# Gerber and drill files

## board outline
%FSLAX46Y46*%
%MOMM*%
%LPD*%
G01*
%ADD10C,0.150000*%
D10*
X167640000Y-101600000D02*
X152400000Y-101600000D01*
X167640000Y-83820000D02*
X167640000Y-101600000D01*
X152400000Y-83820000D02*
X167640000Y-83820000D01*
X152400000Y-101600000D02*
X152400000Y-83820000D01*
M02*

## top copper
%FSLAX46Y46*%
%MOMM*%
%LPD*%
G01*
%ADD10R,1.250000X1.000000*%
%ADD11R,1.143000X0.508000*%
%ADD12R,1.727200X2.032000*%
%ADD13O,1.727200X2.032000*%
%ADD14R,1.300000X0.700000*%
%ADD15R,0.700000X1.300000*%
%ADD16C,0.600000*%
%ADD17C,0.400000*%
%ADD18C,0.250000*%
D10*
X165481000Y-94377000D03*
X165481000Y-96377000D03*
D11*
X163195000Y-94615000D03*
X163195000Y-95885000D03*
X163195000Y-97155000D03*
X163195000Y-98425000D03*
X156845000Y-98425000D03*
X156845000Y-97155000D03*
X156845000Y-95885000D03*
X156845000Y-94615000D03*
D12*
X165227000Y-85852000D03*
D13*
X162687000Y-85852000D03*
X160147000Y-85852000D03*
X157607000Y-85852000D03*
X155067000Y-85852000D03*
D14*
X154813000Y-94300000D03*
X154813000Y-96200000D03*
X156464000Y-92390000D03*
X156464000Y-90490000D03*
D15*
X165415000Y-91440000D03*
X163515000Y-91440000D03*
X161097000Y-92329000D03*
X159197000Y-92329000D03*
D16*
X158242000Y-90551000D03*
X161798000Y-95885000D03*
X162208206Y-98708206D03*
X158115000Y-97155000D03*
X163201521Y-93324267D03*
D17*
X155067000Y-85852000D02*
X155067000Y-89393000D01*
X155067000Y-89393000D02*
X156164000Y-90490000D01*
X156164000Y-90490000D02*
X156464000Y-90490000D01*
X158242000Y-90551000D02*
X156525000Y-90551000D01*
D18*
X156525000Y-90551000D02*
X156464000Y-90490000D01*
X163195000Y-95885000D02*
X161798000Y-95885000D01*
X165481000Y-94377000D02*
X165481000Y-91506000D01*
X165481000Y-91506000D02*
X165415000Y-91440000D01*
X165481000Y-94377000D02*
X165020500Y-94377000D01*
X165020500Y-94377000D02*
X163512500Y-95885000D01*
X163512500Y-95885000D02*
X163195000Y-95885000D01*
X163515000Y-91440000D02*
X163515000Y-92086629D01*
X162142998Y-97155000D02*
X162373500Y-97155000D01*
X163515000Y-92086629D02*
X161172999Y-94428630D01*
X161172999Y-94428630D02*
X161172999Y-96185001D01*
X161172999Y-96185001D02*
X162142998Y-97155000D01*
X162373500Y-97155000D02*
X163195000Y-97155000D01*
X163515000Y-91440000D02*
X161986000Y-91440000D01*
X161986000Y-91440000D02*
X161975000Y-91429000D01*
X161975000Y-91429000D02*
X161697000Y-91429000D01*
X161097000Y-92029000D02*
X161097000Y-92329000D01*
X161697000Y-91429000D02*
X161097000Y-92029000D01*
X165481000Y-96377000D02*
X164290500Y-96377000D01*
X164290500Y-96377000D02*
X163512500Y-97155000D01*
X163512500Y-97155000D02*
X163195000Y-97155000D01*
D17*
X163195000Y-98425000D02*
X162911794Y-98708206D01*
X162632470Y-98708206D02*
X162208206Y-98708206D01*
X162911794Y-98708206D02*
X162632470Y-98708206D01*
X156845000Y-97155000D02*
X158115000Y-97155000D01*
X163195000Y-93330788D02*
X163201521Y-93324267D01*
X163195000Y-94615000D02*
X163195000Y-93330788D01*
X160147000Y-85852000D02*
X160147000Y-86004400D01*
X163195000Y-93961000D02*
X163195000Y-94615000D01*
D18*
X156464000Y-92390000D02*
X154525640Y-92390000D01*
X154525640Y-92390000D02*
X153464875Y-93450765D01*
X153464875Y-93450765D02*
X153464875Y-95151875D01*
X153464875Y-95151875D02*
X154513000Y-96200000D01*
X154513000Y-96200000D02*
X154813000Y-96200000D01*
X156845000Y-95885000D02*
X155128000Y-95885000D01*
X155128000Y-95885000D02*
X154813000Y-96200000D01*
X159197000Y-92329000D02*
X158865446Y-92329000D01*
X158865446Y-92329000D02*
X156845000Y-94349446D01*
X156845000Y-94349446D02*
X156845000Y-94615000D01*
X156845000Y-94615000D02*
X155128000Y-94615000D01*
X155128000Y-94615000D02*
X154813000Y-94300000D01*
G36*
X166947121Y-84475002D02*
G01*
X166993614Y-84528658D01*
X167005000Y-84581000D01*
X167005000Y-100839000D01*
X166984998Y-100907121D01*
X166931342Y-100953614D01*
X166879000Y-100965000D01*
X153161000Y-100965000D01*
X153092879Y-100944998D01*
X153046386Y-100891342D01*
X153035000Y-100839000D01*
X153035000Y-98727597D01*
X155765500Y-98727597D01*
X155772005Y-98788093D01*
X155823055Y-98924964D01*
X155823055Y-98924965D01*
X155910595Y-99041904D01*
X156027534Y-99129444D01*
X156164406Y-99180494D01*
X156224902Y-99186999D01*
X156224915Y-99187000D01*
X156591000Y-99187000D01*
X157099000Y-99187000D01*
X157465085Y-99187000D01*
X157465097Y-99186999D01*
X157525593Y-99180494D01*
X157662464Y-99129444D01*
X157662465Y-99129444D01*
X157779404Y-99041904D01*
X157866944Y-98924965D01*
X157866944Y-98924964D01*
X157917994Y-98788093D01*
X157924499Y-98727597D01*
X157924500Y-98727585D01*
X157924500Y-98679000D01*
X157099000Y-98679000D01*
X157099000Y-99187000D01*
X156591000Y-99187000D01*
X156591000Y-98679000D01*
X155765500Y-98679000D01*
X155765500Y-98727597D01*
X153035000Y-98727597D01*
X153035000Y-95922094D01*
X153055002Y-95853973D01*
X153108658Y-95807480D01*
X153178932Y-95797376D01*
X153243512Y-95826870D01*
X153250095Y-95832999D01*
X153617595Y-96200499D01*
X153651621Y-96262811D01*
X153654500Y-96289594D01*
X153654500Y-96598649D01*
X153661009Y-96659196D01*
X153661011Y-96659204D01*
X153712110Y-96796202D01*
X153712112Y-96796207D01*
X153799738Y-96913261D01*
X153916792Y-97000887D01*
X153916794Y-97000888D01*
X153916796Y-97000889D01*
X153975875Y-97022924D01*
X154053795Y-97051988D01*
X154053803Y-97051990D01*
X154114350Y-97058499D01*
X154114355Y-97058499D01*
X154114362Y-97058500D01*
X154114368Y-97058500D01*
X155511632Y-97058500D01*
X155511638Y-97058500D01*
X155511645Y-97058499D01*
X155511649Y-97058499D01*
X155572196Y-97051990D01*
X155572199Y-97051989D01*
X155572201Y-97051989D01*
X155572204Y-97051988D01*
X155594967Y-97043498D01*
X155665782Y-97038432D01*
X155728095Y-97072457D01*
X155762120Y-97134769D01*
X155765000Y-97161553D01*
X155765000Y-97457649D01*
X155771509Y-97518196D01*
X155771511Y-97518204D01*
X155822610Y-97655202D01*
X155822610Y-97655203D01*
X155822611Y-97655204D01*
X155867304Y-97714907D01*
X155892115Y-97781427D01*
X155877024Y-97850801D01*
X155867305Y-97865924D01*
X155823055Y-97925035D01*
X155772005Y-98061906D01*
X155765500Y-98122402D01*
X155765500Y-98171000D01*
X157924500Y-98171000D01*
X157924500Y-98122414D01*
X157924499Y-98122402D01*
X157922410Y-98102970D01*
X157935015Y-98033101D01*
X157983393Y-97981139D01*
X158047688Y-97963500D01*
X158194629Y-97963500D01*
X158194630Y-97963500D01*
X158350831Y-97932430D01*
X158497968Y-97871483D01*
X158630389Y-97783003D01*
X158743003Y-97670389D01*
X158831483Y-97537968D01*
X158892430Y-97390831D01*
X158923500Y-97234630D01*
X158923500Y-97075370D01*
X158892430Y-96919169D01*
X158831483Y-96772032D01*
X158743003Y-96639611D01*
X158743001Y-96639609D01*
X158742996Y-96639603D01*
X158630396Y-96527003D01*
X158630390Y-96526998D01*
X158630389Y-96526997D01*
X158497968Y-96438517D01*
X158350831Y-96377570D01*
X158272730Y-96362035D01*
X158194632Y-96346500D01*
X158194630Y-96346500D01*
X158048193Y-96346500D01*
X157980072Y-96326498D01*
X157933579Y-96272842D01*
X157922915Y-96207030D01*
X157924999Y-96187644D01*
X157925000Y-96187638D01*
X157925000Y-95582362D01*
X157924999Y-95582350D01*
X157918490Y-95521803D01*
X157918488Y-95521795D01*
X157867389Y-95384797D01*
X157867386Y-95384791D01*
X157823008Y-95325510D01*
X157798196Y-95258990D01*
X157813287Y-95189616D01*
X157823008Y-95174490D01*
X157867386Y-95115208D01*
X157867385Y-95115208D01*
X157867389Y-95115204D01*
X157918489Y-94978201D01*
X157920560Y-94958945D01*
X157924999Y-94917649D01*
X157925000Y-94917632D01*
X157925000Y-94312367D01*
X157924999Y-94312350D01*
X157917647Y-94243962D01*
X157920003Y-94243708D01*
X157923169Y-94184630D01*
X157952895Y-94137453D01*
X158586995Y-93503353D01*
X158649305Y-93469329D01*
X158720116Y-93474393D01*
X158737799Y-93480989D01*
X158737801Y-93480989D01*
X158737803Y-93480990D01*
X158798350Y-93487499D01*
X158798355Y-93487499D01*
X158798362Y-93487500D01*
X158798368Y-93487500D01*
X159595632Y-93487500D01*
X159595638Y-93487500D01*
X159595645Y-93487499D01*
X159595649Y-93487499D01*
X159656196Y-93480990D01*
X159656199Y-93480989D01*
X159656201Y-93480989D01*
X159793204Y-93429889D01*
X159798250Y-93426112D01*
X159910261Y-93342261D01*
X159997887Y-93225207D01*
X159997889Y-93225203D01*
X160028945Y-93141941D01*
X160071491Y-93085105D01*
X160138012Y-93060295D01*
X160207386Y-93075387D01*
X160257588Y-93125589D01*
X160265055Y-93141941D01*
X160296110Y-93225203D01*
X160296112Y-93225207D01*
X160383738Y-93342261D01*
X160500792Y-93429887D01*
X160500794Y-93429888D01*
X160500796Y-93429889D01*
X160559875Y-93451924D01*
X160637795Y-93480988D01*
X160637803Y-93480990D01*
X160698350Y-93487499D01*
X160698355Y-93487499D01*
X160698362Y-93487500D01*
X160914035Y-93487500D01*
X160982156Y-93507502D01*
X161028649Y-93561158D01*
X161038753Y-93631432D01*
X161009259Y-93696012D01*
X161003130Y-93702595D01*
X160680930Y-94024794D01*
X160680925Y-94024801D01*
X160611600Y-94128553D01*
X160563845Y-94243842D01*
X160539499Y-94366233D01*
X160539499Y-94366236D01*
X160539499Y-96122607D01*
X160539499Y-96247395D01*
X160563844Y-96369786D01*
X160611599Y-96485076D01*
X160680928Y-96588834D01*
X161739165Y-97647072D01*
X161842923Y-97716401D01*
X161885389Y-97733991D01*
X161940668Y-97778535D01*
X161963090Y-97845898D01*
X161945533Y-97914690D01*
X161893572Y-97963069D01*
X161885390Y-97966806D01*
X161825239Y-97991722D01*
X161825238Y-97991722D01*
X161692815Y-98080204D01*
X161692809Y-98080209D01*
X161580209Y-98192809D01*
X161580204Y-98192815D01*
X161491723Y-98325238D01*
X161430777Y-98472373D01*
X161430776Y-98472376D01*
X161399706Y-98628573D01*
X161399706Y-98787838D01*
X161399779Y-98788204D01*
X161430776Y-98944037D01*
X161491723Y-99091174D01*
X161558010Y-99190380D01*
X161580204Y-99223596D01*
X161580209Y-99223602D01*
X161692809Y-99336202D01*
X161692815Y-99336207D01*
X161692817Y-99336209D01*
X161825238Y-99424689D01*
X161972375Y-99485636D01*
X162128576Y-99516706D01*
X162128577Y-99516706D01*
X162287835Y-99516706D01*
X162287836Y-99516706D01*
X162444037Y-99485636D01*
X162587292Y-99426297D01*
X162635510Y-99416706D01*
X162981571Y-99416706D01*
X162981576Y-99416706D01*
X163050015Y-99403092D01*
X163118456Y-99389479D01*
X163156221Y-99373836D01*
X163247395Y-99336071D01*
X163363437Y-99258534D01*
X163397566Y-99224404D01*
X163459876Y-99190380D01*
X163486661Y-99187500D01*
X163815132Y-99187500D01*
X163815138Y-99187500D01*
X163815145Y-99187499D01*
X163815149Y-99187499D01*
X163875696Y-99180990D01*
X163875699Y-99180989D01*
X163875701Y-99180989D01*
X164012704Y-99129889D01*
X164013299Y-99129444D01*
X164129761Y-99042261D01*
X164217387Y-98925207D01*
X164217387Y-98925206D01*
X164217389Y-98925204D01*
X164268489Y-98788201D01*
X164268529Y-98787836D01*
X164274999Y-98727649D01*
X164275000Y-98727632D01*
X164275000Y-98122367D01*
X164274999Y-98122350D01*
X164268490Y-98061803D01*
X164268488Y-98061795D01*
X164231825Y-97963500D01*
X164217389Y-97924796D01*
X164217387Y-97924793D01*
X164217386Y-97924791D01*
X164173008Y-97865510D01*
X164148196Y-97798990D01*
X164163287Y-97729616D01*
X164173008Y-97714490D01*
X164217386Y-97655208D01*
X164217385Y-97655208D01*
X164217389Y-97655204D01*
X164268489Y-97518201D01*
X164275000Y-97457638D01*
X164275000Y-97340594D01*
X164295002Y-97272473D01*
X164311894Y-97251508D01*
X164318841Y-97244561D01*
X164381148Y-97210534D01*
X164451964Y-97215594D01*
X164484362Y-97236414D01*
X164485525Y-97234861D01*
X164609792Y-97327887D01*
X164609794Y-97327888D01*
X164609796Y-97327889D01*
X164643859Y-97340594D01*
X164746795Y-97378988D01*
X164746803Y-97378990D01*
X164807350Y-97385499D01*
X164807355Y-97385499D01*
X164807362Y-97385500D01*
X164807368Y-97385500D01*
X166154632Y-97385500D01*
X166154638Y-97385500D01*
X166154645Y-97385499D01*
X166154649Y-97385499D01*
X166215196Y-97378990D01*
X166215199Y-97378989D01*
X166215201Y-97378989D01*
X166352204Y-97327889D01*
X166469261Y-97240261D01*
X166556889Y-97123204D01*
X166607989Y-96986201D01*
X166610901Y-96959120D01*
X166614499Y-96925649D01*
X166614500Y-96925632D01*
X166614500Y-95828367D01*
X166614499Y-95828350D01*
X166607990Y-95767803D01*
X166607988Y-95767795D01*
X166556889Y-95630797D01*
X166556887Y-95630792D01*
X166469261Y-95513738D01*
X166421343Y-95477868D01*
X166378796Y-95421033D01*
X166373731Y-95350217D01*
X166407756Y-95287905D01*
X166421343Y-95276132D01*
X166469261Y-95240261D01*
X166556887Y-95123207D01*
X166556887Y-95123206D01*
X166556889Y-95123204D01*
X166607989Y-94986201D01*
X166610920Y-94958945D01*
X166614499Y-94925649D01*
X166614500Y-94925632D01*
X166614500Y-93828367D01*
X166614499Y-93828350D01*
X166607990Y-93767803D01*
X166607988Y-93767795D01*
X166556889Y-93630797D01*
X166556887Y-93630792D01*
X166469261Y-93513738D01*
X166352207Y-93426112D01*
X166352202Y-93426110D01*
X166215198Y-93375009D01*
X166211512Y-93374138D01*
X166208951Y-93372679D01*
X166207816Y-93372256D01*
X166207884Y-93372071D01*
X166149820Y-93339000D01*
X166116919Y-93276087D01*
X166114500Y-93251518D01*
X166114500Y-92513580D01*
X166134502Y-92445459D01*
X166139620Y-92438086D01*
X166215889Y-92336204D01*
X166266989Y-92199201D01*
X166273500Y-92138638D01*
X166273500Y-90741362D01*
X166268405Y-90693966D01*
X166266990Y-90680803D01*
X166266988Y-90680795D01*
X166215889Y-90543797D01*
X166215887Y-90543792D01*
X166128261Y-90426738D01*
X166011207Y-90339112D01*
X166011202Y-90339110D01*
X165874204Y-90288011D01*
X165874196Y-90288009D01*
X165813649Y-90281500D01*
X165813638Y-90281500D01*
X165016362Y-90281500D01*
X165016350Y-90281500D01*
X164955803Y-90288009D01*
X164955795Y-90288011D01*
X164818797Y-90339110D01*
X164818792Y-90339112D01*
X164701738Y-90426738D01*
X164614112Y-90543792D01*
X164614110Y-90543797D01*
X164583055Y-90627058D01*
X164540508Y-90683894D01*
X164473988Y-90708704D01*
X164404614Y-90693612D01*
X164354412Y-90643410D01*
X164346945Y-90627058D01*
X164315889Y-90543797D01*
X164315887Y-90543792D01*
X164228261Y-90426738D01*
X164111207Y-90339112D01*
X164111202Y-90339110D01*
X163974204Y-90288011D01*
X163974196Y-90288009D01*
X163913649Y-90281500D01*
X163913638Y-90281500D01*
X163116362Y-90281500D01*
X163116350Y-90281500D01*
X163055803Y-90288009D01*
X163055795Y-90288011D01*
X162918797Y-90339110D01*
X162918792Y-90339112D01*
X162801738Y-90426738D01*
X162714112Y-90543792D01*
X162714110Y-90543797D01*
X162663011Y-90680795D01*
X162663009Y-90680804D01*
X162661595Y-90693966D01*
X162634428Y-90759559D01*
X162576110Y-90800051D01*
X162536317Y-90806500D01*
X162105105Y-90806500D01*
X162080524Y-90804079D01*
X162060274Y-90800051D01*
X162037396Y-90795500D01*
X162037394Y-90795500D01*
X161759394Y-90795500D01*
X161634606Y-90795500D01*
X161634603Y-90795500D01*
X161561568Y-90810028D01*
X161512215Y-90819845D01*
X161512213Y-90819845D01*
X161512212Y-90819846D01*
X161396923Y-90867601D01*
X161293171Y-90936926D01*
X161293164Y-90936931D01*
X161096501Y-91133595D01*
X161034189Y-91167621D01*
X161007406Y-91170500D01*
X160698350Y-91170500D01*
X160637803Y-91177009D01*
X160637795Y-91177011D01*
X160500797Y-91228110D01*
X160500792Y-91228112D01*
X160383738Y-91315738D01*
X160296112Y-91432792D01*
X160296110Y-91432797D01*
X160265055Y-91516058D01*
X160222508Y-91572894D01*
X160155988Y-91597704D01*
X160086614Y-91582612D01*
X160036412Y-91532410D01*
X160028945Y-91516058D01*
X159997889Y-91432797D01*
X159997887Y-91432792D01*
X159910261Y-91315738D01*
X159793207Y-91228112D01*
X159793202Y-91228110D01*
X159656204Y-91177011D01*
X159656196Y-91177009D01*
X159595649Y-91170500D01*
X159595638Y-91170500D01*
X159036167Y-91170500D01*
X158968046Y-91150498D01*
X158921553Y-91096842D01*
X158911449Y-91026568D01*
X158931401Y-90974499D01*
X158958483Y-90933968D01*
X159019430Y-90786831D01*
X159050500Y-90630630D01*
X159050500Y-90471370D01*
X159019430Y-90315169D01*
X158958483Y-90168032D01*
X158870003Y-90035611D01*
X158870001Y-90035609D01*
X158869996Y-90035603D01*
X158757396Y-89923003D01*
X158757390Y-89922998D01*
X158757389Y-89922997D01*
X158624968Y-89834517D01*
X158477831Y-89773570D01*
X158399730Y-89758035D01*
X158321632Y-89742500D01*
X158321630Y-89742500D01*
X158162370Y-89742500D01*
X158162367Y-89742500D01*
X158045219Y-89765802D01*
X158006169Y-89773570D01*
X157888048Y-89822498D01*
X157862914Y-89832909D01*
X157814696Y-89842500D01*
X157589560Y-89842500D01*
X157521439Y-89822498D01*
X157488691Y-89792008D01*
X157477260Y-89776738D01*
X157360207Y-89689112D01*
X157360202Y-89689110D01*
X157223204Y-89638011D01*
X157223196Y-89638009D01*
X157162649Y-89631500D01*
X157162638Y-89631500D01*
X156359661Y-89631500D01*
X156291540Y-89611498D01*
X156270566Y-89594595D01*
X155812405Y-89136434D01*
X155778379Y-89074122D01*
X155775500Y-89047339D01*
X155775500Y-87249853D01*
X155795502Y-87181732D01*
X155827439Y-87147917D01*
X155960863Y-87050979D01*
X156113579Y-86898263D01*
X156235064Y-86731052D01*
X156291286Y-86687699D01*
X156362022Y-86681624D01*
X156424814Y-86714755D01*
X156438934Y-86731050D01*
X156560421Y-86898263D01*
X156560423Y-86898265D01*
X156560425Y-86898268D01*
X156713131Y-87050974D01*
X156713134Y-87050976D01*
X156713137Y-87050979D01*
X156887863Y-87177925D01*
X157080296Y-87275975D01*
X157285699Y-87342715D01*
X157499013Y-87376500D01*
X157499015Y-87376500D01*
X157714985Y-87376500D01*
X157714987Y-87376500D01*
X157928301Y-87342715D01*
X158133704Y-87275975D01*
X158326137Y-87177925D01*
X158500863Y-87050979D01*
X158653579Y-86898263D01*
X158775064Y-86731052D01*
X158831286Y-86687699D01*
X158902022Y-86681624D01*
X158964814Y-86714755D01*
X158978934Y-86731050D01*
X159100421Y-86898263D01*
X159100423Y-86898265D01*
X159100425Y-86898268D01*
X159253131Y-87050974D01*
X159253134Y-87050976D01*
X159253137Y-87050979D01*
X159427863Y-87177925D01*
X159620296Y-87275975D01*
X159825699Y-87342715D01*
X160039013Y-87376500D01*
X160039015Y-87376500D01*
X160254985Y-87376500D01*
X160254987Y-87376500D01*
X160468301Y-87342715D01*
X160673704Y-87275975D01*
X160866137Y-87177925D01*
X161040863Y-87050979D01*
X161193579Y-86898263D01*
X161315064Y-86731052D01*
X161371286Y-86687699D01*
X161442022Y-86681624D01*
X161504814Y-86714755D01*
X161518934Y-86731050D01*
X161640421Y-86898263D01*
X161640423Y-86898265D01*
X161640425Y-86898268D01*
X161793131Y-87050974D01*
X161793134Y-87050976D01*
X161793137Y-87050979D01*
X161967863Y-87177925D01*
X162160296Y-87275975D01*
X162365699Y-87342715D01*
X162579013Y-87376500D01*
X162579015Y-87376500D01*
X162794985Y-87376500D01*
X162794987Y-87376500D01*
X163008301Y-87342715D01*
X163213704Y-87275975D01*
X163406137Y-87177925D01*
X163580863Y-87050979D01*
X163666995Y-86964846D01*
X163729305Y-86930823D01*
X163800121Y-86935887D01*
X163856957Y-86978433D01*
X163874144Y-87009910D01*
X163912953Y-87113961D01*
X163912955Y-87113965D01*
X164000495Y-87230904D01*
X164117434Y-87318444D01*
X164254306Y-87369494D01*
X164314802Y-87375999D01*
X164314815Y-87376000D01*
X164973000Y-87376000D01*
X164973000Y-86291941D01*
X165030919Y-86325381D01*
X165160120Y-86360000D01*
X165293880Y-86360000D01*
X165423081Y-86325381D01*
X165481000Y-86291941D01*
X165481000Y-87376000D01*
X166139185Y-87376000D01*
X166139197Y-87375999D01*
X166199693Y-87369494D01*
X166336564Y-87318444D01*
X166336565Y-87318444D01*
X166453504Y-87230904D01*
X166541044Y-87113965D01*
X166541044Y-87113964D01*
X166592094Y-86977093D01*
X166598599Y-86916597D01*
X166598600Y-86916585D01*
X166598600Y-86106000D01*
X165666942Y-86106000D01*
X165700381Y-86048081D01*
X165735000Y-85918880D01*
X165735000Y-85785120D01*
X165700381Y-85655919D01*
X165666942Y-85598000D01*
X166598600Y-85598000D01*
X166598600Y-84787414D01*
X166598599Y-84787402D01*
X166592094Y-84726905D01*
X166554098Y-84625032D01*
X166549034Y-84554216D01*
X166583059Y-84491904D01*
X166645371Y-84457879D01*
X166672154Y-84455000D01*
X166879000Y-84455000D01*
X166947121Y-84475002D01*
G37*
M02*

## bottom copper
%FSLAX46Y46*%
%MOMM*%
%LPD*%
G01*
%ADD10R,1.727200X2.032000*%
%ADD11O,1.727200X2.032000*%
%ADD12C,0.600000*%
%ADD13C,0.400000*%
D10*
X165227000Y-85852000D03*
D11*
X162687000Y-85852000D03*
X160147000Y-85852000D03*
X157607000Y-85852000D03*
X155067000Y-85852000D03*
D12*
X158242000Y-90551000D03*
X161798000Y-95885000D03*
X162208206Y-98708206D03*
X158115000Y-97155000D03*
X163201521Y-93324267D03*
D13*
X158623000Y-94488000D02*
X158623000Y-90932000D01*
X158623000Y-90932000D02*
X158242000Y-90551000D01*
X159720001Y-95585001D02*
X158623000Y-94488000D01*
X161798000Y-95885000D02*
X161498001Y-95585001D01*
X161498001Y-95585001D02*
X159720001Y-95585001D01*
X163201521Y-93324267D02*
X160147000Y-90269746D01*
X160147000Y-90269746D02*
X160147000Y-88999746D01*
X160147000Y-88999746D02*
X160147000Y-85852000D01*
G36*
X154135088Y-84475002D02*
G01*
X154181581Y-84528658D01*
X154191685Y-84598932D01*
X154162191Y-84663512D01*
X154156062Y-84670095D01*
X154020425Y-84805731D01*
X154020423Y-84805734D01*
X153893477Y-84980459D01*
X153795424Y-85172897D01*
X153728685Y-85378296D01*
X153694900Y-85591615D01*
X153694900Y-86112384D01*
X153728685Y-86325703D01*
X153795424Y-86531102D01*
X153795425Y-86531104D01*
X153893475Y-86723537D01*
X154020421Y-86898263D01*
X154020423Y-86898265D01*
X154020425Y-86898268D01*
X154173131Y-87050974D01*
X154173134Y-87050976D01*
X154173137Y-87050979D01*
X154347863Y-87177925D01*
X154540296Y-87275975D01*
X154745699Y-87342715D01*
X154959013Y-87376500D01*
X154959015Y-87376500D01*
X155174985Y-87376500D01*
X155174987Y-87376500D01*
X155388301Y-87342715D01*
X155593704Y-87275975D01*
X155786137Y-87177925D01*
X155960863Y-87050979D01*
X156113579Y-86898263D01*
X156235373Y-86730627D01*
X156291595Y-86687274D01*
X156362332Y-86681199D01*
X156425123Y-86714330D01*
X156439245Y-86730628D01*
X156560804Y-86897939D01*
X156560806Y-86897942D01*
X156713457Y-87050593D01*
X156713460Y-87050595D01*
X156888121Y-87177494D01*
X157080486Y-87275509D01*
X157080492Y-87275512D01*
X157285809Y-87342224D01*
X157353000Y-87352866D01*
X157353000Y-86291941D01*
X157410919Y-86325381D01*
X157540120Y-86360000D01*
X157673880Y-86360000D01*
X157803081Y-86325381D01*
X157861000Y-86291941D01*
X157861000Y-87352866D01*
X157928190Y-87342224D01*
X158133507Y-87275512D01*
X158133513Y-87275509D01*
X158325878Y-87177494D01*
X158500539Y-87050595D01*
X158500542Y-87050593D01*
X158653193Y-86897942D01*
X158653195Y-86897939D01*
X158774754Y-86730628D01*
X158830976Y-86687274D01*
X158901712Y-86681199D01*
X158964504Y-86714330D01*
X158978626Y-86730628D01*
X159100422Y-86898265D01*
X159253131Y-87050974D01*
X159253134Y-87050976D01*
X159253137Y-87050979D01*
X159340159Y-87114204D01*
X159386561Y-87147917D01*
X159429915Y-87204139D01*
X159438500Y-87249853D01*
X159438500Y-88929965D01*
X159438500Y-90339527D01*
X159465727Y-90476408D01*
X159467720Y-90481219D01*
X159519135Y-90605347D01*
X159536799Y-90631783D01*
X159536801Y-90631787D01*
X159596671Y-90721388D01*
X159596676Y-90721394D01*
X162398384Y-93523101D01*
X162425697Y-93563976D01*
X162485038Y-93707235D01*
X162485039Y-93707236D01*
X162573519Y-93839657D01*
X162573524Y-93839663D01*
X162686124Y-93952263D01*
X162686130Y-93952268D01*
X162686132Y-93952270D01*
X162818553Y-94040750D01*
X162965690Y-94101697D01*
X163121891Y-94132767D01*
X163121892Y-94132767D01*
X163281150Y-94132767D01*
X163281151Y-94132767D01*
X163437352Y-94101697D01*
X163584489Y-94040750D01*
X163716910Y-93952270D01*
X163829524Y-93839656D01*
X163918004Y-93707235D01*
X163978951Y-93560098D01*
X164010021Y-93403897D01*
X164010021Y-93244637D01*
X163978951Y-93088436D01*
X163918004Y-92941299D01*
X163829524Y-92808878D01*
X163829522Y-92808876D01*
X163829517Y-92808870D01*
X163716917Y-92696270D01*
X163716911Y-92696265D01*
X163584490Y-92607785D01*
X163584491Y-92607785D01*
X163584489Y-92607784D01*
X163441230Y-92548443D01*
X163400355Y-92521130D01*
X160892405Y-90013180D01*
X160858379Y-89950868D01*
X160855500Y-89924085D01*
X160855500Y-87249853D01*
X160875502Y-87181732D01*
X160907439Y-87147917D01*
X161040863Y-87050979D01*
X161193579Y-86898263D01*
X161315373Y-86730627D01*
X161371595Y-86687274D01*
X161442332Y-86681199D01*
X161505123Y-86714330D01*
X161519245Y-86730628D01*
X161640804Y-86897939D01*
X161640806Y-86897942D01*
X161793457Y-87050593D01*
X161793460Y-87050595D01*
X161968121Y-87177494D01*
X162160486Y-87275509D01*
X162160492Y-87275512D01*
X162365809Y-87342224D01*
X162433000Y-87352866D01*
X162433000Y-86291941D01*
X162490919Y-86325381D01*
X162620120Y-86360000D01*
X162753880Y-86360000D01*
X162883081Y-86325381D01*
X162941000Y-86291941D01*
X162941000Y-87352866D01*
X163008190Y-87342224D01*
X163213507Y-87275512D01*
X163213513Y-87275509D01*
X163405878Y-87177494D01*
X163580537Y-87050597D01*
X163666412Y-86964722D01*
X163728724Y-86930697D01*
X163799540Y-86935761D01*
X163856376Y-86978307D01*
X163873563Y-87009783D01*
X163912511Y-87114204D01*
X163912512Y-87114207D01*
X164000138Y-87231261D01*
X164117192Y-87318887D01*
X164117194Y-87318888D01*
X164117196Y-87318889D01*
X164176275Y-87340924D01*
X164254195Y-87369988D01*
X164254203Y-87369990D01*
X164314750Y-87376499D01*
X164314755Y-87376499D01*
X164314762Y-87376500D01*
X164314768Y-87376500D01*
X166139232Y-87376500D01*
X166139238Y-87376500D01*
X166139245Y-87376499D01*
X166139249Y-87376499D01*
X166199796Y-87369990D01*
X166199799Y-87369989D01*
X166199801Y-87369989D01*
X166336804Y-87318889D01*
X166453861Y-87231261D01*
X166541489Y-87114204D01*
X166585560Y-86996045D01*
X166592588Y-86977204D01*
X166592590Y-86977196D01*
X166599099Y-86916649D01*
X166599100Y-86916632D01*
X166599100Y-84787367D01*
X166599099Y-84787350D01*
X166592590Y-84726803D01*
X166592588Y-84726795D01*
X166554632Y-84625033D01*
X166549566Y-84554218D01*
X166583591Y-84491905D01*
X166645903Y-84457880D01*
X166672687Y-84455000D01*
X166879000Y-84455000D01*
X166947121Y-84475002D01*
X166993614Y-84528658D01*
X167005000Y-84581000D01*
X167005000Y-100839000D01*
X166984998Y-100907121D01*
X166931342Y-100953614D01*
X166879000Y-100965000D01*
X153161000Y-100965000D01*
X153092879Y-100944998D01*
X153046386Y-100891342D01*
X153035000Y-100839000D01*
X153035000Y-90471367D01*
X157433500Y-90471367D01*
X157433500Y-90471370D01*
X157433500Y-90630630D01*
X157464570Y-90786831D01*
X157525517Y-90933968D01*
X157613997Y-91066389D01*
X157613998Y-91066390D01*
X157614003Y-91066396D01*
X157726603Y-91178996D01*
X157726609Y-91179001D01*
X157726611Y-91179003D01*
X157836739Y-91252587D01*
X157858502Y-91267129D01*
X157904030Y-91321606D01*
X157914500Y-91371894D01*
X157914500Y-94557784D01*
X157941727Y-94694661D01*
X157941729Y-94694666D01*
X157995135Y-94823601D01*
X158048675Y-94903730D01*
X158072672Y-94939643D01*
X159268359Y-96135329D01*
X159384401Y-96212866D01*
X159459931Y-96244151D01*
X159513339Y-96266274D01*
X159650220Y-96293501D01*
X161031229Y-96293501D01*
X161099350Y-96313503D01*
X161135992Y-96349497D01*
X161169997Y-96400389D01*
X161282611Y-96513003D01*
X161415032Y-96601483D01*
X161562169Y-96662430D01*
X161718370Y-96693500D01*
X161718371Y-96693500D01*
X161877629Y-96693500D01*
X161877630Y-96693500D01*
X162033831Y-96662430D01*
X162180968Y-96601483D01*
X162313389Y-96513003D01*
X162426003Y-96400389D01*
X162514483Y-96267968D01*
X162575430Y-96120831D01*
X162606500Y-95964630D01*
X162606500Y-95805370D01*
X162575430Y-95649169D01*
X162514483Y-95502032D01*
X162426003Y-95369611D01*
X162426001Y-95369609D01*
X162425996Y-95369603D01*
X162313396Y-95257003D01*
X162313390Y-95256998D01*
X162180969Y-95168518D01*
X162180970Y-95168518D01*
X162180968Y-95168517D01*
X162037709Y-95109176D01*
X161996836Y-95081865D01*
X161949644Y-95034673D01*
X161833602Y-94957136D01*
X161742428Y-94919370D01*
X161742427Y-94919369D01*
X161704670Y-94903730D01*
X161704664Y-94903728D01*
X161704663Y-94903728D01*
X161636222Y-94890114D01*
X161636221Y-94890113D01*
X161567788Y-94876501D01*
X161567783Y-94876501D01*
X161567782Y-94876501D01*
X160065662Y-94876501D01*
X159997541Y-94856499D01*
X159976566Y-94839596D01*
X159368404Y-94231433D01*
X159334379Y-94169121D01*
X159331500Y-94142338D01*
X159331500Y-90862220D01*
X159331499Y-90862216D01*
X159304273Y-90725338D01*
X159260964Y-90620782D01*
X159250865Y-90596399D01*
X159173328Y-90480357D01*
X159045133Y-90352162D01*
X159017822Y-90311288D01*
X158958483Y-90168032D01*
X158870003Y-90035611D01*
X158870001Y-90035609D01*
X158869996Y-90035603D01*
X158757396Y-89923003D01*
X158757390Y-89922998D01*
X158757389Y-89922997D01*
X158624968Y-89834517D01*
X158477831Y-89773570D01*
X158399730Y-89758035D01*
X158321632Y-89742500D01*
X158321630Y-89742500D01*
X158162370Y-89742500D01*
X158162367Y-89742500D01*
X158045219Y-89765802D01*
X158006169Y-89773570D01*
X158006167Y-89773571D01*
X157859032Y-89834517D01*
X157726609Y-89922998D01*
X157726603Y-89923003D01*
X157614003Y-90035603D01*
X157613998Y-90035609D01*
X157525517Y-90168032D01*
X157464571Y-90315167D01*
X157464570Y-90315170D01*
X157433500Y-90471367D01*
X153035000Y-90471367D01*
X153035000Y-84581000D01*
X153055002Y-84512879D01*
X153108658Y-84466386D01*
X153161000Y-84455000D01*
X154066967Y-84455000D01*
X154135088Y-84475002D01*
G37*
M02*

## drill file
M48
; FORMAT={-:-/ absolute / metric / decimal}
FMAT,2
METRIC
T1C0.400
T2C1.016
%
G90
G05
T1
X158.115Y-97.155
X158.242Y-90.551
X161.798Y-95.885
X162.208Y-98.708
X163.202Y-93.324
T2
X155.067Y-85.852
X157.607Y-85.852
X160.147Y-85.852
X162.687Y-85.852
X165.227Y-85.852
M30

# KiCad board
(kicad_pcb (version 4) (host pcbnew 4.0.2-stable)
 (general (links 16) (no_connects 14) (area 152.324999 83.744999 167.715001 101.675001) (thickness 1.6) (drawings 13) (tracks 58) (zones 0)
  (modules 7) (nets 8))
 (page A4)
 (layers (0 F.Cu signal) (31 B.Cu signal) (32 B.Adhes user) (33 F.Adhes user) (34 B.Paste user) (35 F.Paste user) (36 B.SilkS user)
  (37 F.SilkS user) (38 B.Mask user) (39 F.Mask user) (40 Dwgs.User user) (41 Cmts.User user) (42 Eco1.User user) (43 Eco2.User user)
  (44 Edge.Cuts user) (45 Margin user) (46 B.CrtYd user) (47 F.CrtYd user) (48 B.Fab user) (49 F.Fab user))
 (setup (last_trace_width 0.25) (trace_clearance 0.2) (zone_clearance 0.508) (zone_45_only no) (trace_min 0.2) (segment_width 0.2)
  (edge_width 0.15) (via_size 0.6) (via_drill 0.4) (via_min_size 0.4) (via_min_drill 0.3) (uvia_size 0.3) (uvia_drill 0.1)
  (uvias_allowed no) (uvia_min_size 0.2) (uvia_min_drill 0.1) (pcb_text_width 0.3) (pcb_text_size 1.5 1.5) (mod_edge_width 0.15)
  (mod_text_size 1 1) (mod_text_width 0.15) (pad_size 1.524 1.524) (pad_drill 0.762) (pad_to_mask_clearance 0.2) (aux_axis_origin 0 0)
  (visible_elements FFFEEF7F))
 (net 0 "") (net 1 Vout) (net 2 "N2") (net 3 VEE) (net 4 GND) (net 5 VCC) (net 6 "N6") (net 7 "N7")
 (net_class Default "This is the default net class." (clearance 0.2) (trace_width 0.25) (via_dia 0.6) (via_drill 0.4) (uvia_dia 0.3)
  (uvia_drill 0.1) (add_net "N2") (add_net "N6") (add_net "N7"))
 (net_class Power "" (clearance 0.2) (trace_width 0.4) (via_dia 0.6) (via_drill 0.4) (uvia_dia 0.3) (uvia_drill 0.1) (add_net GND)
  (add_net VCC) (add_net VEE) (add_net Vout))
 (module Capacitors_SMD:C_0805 (layer F.Cu) (at 165.481 95.377 270)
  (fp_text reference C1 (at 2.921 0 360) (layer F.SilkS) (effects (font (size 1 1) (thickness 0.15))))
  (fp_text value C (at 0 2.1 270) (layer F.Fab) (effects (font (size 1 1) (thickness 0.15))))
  (pad 1 smd rect (at -1 0 270) (size 1 1.25) (layers F.Cu F.Paste F.Mask) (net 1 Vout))
  (pad 2 smd rect (at 1 0 270) (size 1 1.25) (layers F.Cu F.Paste F.Mask) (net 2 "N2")))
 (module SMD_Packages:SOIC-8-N (layer F.Cu) (at 160.02 96.52 270)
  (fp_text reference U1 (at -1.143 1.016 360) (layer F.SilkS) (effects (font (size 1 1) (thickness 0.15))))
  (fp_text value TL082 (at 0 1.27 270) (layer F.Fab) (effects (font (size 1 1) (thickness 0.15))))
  (pad 8 smd rect (at -1.905 -3.175 270) (size 0.508 1.143) (layers F.Cu F.Paste F.Mask) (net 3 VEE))
  (pad 7 smd rect (at -0.635 -3.175 270) (size 0.508 1.143) (layers F.Cu F.Paste F.Mask) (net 1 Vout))
  (pad 6 smd rect (at 0.635 -3.175 270) (size 0.508 1.143) (layers F.Cu F.Paste F.Mask) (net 2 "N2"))
  (pad 5 smd rect (at 1.905 -3.175 270) (size 0.508 1.143) (layers F.Cu F.Paste F.Mask) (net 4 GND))
  (pad 4 smd rect (at 1.905 3.175 270) (size 0.508 1.143) (layers F.Cu F.Paste F.Mask) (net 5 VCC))
  (pad 3 smd rect (at 0.635 3.175 270) (size 0.508 1.143) (layers F.Cu F.Paste F.Mask) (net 4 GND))
  (pad 2 smd rect (at -0.635 3.175 270) (size 0.508 1.143) (layers F.Cu F.Paste F.Mask) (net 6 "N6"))
  (pad 1 smd rect (at -1.905 3.175 270) (size 0.508 1.143) (layers F.Cu F.Paste F.Mask) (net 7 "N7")))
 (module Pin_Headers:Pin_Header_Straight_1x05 (layer F.Cu) (at 165.227 85.852 270)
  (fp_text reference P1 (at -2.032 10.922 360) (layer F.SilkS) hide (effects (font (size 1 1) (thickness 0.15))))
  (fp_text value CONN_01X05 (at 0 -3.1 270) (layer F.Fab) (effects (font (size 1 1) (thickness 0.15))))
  (pad 1 thru_hole rect (at 0 0 270) (size 2.032 1.7272) (drill 1.016) (layers *.Cu *.Mask F.SilkS) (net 5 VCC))
  (pad 2 thru_hole oval (at 0 2.54 270) (size 2.032 1.7272) (drill 1.016) (layers *.Cu *.Mask F.SilkS) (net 4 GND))
  (pad 3 thru_hole oval (at 0 5.08 270) (size 2.032 1.7272) (drill 1.016) (layers *.Cu *.Mask F.SilkS) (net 3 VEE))
  (pad 4 thru_hole oval (at 0 7.62 270) (size 2.032 1.7272) (drill 1.016) (layers *.Cu *.Mask F.SilkS) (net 4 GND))
  (pad 5 thru_hole oval (at 0 10.16 270) (size 2.032 1.7272) (drill 1.016) (layers *.Cu *.Mask F.SilkS) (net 1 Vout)))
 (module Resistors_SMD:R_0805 (layer F.Cu) (at 154.813 95.25 270)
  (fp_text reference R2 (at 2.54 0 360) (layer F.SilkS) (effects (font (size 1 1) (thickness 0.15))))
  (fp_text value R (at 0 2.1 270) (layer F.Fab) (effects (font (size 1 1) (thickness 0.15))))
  (pad 1 smd rect (at -0.95 0 270) (size 0.7 1.3) (layers F.Cu F.Paste F.Mask) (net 7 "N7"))
  (pad 2 smd rect (at 0.95 0 270) (size 0.7 1.3) (layers F.Cu F.Paste F.Mask) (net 6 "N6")))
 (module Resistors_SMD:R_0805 (layer F.Cu) (at 156.464 91.44 90)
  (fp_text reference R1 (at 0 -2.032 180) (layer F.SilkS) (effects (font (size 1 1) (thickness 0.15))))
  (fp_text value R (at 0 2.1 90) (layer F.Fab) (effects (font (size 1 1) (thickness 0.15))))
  (pad 1 smd rect (at -0.95 0 90) (size 0.7 1.3) (layers F.Cu F.Paste F.Mask) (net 6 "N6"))
  (pad 2 smd rect (at 0.95 0 90) (size 0.7 1.3) (layers F.Cu F.Paste F.Mask) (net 1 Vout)))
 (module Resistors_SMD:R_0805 (layer F.Cu) (at 164.465 91.44 180)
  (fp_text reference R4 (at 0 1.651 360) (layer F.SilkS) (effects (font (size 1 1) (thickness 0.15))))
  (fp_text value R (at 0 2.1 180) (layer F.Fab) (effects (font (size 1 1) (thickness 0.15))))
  (pad 1 smd rect (at -0.95 0 180) (size 0.7 1.3) (layers F.Cu F.Paste F.Mask) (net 1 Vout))
  (pad 2 smd rect (at 0.95 0 180) (size 0.7 1.3) (layers F.Cu F.Paste F.Mask) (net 2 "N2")))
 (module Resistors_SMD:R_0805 (layer F.Cu) (at 160.147 92.329 180)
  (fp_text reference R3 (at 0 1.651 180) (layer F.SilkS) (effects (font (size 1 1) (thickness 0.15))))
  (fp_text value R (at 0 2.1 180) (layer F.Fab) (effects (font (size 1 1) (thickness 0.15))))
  (pad 1 smd rect (at -0.95 0 180) (size 0.7 1.3) (layers F.Cu F.Paste F.Mask) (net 2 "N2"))
  (pad 2 smd rect (at 0.95 0 180) (size 0.7 1.3) (layers F.Cu F.Paste F.Mask) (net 7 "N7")))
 (gr_line (start 167.64 101.6) (end 152.4 101.6) (layer Edge.Cuts) (width 0.15))
 (gr_line (start 167.64 83.82) (end 167.64 101.6) (layer Edge.Cuts) (width 0.15))
 (gr_line (start 152.4 83.82) (end 167.64 83.82) (layer Edge.Cuts) (width 0.15))
 (gr_line (start 152.4 101.6) (end 152.4 83.82) (layer Edge.Cuts) (width 0.15))
 (segment (start 155.067 85.852) (end 155.067 89.393) (width 0.4) (layer F.Cu) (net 1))
 (segment (start 155.067 89.393) (end 156.164 90.49) (width 0.4) (layer F.Cu) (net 1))
 (segment (start 156.164 90.49) (end 156.464 90.49) (width 0.4) (layer F.Cu) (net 1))
 (segment (start 158.242 90.551) (end 156.525 90.551) (width 0.4) (layer F.Cu) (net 1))
 (segment (start 156.525 90.551) (end 156.464 90.49) (width 0.25) (layer F.Cu) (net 1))
 (segment (start 158.623 94.488) (end 158.623 90.932) (width 0.4) (layer B.Cu) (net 1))
 (segment (start 158.623 90.932) (end 158.242 90.551) (width 0.4) (layer B.Cu) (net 1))
 (via (at 158.242 90.551) (size 0.6) (drill 0.4) (layers F.Cu B.Cu) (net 1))
 (segment (start 159.720001 95.585001) (end 158.623 94.488) (width 0.4) (layer B.Cu) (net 1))
 (segment (start 161.798 95.885) (end 161.498001 95.585001) (width 0.4) (layer B.Cu) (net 1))
 (segment (start 161.498001 95.585001) (end 159.720001 95.585001) (width 0.4) (layer B.Cu) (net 1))
 (segment (start 163.195 95.885) (end 161.798 95.885) (width 0.25) (layer F.Cu) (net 1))
 (via (at 161.798 95.885) (size 0.6) (drill 0.4) (layers F.Cu B.Cu) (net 1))
 (segment (start 165.481 94.377) (end 165.481 91.506) (width 0.25) (layer F.Cu) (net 1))
 (segment (start 165.481 91.506) (end 165.415 91.44) (width 0.25) (layer F.Cu) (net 1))
 (segment (start 165.481 94.377) (end 165.0205 94.377) (width 0.25) (layer F.Cu) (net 1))
 (segment (start 165.0205 94.377) (end 163.5125 95.885) (width 0.25) (layer F.Cu) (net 1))
 (segment (start 163.5125 95.885) (end 163.195 95.885) (width 0.25) (layer F.Cu) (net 1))
 (segment (start 163.515 91.44) (end 163.515 92.086629) (width 0.25) (layer F.Cu) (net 2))
 (segment (start 162.142998 97.155) (end 162.3735 97.155) (width 0.25) (layer F.Cu) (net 2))
 (segment (start 163.515 92.086629) (end 161.172999 94.42863) (width 0.25) (layer F.Cu) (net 2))
 (segment (start 161.172999 94.42863) (end 161.172999 96.185001) (width 0.25) (layer F.Cu) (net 2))
 (segment (start 161.172999 96.185001) (end 162.142998 97.155) (width 0.25) (layer F.Cu) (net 2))
 (segment (start 162.3735 97.155) (end 163.195 97.155) (width 0.25) (layer F.Cu) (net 2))
 (segment (start 163.515 91.44) (end 161.986 91.44) (width 0.25) (layer F.Cu) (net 2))
 (segment (start 161.986 91.44) (end 161.975 91.429) (width 0.25) (layer F.Cu) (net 2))
 (segment (start 161.975 91.429) (end 161.697 91.429) (width 0.25) (layer F.Cu) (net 2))
 (segment (start 161.097 92.029) (end 161.097 92.329) (width 0.25) (layer F.Cu) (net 2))
 (segment (start 161.697 91.429) (end 161.097 92.029) (width 0.25) (layer F.Cu) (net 2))
 (segment (start 165.481 96.377) (end 164.2905 96.377) (width 0.25) (layer F.Cu) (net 2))
 (segment (start 164.2905 96.377) (end 163.5125 97.155) (width 0.25) (layer F.Cu) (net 2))
 (segment (start 163.5125 97.155) (end 163.195 97.155) (width 0.25) (layer F.Cu) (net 2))
 (segment (start 163.195 98.425) (end 162.911794 98.708206) (width 0.4) (layer F.Cu) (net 4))
 (via (at 162.208206 98.708206) (size 0.6) (drill 0.4) (layers F.Cu B.Cu) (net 4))
 (segment (start 162.63247 98.708206) (end 162.208206 98.708206) (width 0.4) (layer F.Cu) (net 4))
 (segment (start 162.911794 98.708206) (end 162.63247 98.708206) (width 0.4) (layer F.Cu) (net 4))
 (segment (start 156.845 97.155) (end 158.115 97.155) (width 0.4) (layer F.Cu) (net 4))
 (via (at 158.115 97.155) (size 0.6) (drill 0.4) (layers F.Cu B.Cu) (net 4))
 (segment (start 163.201521 93.324267) (end 160.147 90.269746) (width 0.4) (layer B.Cu) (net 3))
 (segment (start 160.147 90.269746) (end 160.147 88.999746) (width 0.4) (layer B.Cu) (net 3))
 (segment (start 160.147 88.999746) (end 160.147 85.852) (width 0.4) (layer B.Cu) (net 3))
 (segment (start 163.195 93.330788) (end 163.201521 93.324267) (width 0.4) (layer F.Cu) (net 3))
 (segment (start 163.195 94.615) (end 163.195 93.330788) (width 0.4) (layer F.Cu) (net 3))
 (via (at 163.201521 93.324267) (size 0.6) (drill 0.4) (layers F.Cu B.Cu) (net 3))
 (segment (start 160.147 85.852) (end 160.147 86.0044) (width 0.4) (layer F.Cu) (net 3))
 (segment (start 163.195 93.961) (end 163.195 94.615) (width 0.4) (layer F.Cu) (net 3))
 (segment (start 156.464 92.39) (end 154.52564 92.39) (width 0.25) (layer F.Cu) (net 6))
 (segment (start 154.52564 92.39) (end 153.464875 93.450765) (width 0.25) (layer F.Cu) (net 6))
 (segment (start 153.464875 93.450765) (end 153.464875 95.151875) (width 0.25) (layer F.Cu) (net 6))
 (segment (start 153.464875 95.151875) (end 154.513 96.2) (width 0.25) (layer F.Cu) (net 6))
 (segment (start 154.513 96.2) (end 154.813 96.2) (width 0.25) (layer F.Cu) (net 6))
 (segment (start 156.845 95.885) (end 155.128 95.885) (width 0.25) (layer F.Cu) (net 6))
 (segment (start 155.128 95.885) (end 154.813 96.2) (width 0.25) (layer F.Cu) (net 6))
 (segment (start 159.197 92.329) (end 158.865446 92.329) (width 0.25) (layer F.Cu) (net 7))
 (segment (start 158.865446 92.329) (end 156.845 94.349446) (width 0.25) (layer F.Cu) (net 7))
 (segment (start 156.845 94.349446) (end 156.845 94.615) (width 0.25) (layer F.Cu) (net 7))
 (segment (start 156.845 94.615) (end 155.128 94.615) (width 0.25) (layer F.Cu) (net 7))
 (segment (start 155.128 94.615) (end 154.813 94.3) (width 0.25) (layer F.Cu) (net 7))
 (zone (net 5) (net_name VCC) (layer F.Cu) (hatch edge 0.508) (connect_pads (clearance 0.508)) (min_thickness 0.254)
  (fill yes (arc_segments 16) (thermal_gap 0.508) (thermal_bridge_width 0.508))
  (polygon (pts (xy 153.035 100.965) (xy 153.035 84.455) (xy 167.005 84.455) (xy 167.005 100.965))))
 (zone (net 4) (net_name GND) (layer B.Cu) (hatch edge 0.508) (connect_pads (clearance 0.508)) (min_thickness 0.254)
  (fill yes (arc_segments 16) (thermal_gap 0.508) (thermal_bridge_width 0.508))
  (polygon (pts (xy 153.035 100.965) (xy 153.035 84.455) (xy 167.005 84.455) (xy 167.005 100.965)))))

